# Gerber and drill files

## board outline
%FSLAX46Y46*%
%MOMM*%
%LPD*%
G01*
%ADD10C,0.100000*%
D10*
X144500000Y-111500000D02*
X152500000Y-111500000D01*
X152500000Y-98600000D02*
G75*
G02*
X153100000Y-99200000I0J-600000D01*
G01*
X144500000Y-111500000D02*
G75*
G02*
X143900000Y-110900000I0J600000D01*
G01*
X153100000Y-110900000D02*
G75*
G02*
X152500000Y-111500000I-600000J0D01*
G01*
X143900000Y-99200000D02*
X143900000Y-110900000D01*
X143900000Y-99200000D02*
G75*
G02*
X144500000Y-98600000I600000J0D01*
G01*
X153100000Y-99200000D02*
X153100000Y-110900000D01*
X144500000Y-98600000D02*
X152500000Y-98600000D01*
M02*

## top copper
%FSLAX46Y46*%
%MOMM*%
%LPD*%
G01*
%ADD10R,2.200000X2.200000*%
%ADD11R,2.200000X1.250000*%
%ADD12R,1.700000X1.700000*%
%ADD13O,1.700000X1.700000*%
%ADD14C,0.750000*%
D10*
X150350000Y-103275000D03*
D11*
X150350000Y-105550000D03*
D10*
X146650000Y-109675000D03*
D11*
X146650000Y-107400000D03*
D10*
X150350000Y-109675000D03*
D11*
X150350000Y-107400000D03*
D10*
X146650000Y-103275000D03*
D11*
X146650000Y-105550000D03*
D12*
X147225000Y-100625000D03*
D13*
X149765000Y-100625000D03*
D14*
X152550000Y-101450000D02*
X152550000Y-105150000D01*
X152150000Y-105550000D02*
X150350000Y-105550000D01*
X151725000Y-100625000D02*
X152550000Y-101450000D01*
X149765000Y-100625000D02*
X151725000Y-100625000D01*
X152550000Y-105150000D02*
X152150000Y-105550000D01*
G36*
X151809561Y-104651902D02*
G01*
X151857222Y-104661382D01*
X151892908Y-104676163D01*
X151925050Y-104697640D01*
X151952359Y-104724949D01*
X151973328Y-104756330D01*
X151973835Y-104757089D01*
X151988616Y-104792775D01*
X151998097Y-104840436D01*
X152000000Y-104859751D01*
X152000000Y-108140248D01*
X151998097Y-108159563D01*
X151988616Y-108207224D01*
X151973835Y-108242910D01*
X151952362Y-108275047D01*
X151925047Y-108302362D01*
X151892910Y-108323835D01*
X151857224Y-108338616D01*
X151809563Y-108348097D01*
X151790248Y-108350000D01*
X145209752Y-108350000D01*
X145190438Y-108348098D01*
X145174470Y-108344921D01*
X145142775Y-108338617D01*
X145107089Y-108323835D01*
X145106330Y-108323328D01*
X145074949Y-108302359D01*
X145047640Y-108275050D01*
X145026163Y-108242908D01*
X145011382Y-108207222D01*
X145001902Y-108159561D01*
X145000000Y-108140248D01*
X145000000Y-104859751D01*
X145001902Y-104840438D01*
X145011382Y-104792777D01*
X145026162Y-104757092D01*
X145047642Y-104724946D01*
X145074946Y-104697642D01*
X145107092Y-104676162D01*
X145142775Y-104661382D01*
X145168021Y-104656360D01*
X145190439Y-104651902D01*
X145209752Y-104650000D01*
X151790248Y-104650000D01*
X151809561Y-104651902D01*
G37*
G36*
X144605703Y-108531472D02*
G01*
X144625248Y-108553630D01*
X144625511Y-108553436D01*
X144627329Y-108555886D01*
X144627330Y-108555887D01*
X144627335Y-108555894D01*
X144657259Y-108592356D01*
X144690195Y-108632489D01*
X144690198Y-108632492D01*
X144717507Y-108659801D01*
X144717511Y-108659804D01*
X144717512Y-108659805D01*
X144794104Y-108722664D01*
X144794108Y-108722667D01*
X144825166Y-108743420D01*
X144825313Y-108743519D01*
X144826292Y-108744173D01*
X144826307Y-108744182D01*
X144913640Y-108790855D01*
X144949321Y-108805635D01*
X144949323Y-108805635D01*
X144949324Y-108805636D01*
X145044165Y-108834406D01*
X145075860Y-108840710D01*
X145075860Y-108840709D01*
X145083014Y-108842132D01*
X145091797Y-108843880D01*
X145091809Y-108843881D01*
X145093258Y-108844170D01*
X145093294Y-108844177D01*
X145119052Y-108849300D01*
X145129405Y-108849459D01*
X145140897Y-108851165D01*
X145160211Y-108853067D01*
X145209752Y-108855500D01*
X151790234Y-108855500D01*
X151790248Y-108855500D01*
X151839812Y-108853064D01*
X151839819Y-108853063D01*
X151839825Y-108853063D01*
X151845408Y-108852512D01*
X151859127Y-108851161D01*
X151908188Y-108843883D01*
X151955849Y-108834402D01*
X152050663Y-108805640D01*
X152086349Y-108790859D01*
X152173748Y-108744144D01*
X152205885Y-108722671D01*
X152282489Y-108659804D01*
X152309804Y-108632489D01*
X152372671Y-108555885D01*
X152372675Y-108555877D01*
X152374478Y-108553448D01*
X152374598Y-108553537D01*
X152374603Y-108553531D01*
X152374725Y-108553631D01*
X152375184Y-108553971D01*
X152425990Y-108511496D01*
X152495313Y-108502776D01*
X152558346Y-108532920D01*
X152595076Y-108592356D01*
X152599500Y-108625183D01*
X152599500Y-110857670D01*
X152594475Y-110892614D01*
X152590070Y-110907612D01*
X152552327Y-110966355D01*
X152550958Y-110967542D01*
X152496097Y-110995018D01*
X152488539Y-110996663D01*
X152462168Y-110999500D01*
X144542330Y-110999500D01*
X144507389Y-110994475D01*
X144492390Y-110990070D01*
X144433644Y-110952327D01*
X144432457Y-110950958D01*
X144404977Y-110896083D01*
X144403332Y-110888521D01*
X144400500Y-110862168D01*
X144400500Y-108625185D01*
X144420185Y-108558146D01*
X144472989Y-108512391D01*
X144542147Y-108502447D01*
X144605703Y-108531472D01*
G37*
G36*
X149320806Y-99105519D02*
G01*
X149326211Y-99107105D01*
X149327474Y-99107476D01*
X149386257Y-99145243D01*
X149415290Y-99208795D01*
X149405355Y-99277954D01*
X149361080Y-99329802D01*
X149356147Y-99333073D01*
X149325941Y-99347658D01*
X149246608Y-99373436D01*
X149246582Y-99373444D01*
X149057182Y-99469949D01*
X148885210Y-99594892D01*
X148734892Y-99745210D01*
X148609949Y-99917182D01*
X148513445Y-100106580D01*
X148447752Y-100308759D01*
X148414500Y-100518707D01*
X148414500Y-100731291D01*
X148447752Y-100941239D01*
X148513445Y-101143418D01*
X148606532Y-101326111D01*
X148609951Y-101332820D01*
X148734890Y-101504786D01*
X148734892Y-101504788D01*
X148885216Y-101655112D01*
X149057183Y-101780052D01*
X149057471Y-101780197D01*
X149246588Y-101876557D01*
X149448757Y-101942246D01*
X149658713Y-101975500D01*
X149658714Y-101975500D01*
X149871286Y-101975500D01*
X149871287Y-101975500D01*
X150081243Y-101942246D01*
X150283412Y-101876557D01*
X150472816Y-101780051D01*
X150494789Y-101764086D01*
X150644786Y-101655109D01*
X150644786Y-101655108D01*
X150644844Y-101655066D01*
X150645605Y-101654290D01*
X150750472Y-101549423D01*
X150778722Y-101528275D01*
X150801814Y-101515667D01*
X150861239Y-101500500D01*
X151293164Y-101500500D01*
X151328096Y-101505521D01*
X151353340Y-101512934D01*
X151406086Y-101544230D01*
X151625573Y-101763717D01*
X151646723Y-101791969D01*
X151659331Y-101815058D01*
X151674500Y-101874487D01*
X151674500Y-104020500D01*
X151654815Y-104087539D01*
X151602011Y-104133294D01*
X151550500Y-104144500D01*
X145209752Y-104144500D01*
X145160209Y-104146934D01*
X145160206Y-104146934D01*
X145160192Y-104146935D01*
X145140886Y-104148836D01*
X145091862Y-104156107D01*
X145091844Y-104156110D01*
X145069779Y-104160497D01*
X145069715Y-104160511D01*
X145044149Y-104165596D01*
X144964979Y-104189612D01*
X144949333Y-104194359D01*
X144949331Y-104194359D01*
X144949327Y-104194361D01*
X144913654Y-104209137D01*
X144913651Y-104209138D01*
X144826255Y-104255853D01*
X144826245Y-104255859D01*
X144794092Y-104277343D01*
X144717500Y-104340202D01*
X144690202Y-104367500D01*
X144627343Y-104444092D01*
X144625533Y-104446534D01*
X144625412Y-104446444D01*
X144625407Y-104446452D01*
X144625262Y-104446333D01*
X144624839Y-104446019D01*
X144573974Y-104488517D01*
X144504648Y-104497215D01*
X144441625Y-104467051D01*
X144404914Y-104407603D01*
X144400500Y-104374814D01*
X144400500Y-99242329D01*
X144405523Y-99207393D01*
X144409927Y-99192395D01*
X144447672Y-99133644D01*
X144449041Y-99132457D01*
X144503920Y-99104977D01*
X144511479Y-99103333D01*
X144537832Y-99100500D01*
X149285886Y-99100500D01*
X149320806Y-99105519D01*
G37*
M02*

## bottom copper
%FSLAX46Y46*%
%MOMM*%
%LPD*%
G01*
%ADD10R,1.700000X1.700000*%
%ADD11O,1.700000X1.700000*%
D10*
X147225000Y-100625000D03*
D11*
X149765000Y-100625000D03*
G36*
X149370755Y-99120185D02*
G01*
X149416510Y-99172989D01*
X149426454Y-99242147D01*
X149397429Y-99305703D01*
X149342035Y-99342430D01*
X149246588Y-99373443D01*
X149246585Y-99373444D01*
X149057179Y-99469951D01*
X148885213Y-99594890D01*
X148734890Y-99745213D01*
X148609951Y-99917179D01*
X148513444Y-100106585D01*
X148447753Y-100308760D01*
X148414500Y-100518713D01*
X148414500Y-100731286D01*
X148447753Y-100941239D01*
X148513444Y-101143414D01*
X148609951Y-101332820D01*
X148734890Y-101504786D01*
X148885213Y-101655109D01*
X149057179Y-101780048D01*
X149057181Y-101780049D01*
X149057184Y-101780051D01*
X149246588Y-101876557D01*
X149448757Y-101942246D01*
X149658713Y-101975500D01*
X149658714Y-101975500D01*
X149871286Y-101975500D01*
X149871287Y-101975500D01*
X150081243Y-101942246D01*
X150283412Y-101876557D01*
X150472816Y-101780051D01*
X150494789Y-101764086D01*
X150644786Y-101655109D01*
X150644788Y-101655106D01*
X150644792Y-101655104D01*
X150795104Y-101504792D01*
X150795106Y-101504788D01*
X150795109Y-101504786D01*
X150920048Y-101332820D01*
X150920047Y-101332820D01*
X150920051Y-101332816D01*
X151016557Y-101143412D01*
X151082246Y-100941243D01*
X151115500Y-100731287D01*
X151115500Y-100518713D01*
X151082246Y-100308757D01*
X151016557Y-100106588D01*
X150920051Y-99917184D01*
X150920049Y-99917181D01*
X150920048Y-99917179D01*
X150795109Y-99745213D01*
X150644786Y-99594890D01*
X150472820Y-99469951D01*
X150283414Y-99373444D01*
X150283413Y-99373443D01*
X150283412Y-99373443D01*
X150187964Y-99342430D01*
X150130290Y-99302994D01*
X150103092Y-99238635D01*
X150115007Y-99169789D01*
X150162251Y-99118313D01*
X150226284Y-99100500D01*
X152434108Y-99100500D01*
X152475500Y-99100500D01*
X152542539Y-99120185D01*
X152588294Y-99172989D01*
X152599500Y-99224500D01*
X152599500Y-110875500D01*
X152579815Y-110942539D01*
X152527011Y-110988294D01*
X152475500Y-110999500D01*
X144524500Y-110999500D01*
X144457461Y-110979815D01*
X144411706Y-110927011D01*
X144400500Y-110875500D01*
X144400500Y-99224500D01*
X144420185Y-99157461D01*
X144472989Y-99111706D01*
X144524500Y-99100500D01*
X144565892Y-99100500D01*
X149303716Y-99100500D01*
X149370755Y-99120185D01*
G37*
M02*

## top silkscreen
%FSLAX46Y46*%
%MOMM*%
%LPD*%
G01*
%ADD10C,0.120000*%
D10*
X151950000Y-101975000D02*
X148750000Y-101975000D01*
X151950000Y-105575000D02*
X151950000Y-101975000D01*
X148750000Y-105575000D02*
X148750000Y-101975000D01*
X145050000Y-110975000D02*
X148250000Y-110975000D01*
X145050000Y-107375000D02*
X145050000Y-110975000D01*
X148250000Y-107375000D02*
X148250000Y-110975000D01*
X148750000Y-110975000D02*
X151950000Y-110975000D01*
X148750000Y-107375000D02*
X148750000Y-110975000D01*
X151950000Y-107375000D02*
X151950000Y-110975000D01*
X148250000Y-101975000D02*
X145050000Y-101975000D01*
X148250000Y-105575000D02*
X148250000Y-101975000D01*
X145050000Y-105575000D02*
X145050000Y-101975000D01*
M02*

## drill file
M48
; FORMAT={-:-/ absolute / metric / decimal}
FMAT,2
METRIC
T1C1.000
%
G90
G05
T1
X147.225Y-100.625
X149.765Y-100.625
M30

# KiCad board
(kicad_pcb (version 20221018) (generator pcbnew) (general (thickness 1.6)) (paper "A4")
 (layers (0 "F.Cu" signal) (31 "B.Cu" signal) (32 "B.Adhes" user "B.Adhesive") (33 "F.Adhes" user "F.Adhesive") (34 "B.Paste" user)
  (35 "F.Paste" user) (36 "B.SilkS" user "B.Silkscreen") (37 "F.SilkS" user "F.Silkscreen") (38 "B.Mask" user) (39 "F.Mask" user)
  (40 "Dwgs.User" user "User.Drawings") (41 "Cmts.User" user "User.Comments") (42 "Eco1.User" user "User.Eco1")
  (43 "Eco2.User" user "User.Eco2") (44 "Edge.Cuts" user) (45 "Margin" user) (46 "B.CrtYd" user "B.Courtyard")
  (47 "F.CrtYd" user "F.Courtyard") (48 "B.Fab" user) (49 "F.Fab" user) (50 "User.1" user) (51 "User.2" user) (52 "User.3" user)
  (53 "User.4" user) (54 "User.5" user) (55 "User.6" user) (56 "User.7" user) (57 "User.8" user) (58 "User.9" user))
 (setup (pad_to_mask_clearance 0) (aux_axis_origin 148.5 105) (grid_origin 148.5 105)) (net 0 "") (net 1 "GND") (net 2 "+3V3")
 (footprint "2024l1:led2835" (layer "F.Cu") (at 150.35 104.175 -90)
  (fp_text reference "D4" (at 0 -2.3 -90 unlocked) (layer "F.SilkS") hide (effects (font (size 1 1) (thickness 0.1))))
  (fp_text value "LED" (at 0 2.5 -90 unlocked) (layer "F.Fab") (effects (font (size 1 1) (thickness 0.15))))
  (fp_line (start -2.2 -1.6) (end -2.2 1.6) (stroke (width 0.12) (type solid)) (layer "F.SilkS"))
  (fp_line (start 1.4 -1.6) (end -2.2 -1.6) (stroke (width 0.12) (type solid)) (layer "F.SilkS"))
  (fp_line (start 1.4 1.6) (end -2.2 1.6) (stroke (width 0.12) (type solid)) (layer "F.SilkS"))
  (pad "1" smd rect (at -0.9 0 270) (size 2.2 2.2) (layers "F.Cu" "F.Paste" "F.Mask") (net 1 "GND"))
  (pad "2" smd rect (at 1.375 0 270) (size 1.25 2.2) (layers "F.Cu" "F.Paste" "F.Mask") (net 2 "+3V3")))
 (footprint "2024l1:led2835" (layer "F.Cu") (at 146.65 108.775 90)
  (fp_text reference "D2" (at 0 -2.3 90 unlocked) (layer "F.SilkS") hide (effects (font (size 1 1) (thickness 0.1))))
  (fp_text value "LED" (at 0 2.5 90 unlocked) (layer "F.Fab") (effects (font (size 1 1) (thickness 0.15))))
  (fp_line (start -2.2 -1.6) (end -2.2 1.6) (stroke (width 0.12) (type solid)) (layer "F.SilkS"))
  (fp_line (start 1.4 -1.6) (end -2.2 -1.6) (stroke (width 0.12) (type solid)) (layer "F.SilkS"))
  (fp_line (start 1.4 1.6) (end -2.2 1.6) (stroke (width 0.12) (type solid)) (layer "F.SilkS"))
  (pad "1" smd rect (at -0.9 0 90) (size 2.2 2.2) (layers "F.Cu" "F.Paste" "F.Mask") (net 1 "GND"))
  (pad "2" smd rect (at 1.375 0 90) (size 1.25 2.2) (layers "F.Cu" "F.Paste" "F.Mask") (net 2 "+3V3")))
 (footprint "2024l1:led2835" (layer "F.Cu") (at 150.35 108.775 90)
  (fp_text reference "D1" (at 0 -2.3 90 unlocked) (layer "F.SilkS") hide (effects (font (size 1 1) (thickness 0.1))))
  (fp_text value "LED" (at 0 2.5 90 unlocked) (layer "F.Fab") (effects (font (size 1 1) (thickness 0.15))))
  (fp_line (start -2.2 -1.6) (end -2.2 1.6) (stroke (width 0.12) (type solid)) (layer "F.SilkS"))
  (fp_line (start 1.4 -1.6) (end -2.2 -1.6) (stroke (width 0.12) (type solid)) (layer "F.SilkS"))
  (fp_line (start 1.4 1.6) (end -2.2 1.6) (stroke (width 0.12) (type solid)) (layer "F.SilkS"))
  (pad "1" smd rect (at -0.9 0 90) (size 2.2 2.2) (layers "F.Cu" "F.Paste" "F.Mask") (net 1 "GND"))
  (pad "2" smd rect (at 1.375 0 90) (size 1.25 2.2) (layers "F.Cu" "F.Paste" "F.Mask") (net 2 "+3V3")))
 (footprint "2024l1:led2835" (layer "F.Cu") (at 146.65 104.175 -90)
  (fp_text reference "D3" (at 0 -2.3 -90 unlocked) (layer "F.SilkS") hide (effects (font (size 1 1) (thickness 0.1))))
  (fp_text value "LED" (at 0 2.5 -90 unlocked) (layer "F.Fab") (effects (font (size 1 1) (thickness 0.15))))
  (fp_line (start -2.2 -1.6) (end -2.2 1.6) (stroke (width 0.12) (type solid)) (layer "F.SilkS"))
  (fp_line (start 1.4 -1.6) (end -2.2 -1.6) (stroke (width 0.12) (type solid)) (layer "F.SilkS"))
  (fp_line (start 1.4 1.6) (end -2.2 1.6) (stroke (width 0.12) (type solid)) (layer "F.SilkS"))
  (pad "1" smd rect (at -0.9 0 270) (size 2.2 2.2) (layers "F.Cu" "F.Paste" "F.Mask") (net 1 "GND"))
  (pad "2" smd rect (at 1.375 0 270) (size 1.25 2.2) (layers "F.Cu" "F.Paste" "F.Mask") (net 2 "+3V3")))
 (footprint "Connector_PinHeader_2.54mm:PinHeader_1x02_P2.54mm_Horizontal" (layer "B.Cu") (at 147.225 100.625 -90)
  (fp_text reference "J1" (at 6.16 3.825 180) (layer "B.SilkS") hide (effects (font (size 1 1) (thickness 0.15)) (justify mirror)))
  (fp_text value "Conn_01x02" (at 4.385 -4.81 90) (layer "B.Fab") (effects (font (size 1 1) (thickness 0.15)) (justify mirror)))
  (pad "1" thru_hole rect (at 0 0 270) (size 1.7 1.7) (drill 1) (layers "*.Cu" "*.Mask") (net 1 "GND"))
  (pad "2" thru_hole oval (at 0 -2.54 270) (size 1.7 1.7) (drill 1) (layers "*.Cu" "*.Mask") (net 2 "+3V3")))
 (gr_line (start 144.5 111.5) (end 152.5 111.5) (stroke (width 0.1) (type default)) (layer "Edge.Cuts"))
 (gr_arc (start 152.5 98.6) (mid 152.924264 98.775736) (end 153.1 99.2) (stroke (width 0.1) (type default)) (layer "Edge.Cuts"))
 (gr_arc (start 144.5 111.5) (mid 144.075736 111.324264) (end 143.9 110.9) (stroke (width 0.1) (type default)) (layer "Edge.Cuts"))
 (gr_arc (start 153.1 110.9) (mid 152.924264 111.324264) (end 152.5 111.5) (stroke (width 0.1) (type default)) (layer "Edge.Cuts"))
 (gr_line (start 143.9 99.2) (end 143.9 110.9) (stroke (width 0.1) (type default)) (layer "Edge.Cuts"))
 (gr_arc (start 143.9 99.2) (mid 144.075736 98.775736) (end 144.5 98.6) (stroke (width 0.1) (type default)) (layer "Edge.Cuts"))
 (gr_line (start 153.1 99.2) (end 153.1 110.9) (stroke (width 0.1) (type default)) (layer "Edge.Cuts"))
 (gr_line (start 144.5 98.6) (end 152.5 98.6) (stroke (width 0.1) (type default)) (layer "Edge.Cuts"))
 (segment (start 152.55 101.45) (end 152.55 105.15) (width 0.75) (layer "F.Cu") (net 2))
 (segment (start 152.15 105.55) (end 150.35 105.55) (width 0.75) (layer "F.Cu") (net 2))
 (segment (start 151.725 100.625) (end 152.55 101.45) (width 0.75) (layer "F.Cu") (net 2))
 (segment (start 149.765 100.625) (end 151.725 100.625) (width 0.75) (layer "F.Cu") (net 2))
 (segment (start 152.55 105.15) (end 152.15 105.55) (width 0.75) (layer "F.Cu") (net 2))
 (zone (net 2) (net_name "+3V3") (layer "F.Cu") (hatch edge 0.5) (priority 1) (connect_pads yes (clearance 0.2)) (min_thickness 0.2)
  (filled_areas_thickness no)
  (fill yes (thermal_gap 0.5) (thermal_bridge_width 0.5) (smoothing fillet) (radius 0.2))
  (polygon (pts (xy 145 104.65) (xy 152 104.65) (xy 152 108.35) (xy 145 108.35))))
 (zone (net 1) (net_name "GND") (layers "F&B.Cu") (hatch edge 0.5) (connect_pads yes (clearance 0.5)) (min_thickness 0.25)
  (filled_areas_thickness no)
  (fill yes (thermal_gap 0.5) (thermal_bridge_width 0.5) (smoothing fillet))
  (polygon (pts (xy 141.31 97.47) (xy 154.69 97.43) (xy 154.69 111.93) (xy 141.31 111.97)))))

